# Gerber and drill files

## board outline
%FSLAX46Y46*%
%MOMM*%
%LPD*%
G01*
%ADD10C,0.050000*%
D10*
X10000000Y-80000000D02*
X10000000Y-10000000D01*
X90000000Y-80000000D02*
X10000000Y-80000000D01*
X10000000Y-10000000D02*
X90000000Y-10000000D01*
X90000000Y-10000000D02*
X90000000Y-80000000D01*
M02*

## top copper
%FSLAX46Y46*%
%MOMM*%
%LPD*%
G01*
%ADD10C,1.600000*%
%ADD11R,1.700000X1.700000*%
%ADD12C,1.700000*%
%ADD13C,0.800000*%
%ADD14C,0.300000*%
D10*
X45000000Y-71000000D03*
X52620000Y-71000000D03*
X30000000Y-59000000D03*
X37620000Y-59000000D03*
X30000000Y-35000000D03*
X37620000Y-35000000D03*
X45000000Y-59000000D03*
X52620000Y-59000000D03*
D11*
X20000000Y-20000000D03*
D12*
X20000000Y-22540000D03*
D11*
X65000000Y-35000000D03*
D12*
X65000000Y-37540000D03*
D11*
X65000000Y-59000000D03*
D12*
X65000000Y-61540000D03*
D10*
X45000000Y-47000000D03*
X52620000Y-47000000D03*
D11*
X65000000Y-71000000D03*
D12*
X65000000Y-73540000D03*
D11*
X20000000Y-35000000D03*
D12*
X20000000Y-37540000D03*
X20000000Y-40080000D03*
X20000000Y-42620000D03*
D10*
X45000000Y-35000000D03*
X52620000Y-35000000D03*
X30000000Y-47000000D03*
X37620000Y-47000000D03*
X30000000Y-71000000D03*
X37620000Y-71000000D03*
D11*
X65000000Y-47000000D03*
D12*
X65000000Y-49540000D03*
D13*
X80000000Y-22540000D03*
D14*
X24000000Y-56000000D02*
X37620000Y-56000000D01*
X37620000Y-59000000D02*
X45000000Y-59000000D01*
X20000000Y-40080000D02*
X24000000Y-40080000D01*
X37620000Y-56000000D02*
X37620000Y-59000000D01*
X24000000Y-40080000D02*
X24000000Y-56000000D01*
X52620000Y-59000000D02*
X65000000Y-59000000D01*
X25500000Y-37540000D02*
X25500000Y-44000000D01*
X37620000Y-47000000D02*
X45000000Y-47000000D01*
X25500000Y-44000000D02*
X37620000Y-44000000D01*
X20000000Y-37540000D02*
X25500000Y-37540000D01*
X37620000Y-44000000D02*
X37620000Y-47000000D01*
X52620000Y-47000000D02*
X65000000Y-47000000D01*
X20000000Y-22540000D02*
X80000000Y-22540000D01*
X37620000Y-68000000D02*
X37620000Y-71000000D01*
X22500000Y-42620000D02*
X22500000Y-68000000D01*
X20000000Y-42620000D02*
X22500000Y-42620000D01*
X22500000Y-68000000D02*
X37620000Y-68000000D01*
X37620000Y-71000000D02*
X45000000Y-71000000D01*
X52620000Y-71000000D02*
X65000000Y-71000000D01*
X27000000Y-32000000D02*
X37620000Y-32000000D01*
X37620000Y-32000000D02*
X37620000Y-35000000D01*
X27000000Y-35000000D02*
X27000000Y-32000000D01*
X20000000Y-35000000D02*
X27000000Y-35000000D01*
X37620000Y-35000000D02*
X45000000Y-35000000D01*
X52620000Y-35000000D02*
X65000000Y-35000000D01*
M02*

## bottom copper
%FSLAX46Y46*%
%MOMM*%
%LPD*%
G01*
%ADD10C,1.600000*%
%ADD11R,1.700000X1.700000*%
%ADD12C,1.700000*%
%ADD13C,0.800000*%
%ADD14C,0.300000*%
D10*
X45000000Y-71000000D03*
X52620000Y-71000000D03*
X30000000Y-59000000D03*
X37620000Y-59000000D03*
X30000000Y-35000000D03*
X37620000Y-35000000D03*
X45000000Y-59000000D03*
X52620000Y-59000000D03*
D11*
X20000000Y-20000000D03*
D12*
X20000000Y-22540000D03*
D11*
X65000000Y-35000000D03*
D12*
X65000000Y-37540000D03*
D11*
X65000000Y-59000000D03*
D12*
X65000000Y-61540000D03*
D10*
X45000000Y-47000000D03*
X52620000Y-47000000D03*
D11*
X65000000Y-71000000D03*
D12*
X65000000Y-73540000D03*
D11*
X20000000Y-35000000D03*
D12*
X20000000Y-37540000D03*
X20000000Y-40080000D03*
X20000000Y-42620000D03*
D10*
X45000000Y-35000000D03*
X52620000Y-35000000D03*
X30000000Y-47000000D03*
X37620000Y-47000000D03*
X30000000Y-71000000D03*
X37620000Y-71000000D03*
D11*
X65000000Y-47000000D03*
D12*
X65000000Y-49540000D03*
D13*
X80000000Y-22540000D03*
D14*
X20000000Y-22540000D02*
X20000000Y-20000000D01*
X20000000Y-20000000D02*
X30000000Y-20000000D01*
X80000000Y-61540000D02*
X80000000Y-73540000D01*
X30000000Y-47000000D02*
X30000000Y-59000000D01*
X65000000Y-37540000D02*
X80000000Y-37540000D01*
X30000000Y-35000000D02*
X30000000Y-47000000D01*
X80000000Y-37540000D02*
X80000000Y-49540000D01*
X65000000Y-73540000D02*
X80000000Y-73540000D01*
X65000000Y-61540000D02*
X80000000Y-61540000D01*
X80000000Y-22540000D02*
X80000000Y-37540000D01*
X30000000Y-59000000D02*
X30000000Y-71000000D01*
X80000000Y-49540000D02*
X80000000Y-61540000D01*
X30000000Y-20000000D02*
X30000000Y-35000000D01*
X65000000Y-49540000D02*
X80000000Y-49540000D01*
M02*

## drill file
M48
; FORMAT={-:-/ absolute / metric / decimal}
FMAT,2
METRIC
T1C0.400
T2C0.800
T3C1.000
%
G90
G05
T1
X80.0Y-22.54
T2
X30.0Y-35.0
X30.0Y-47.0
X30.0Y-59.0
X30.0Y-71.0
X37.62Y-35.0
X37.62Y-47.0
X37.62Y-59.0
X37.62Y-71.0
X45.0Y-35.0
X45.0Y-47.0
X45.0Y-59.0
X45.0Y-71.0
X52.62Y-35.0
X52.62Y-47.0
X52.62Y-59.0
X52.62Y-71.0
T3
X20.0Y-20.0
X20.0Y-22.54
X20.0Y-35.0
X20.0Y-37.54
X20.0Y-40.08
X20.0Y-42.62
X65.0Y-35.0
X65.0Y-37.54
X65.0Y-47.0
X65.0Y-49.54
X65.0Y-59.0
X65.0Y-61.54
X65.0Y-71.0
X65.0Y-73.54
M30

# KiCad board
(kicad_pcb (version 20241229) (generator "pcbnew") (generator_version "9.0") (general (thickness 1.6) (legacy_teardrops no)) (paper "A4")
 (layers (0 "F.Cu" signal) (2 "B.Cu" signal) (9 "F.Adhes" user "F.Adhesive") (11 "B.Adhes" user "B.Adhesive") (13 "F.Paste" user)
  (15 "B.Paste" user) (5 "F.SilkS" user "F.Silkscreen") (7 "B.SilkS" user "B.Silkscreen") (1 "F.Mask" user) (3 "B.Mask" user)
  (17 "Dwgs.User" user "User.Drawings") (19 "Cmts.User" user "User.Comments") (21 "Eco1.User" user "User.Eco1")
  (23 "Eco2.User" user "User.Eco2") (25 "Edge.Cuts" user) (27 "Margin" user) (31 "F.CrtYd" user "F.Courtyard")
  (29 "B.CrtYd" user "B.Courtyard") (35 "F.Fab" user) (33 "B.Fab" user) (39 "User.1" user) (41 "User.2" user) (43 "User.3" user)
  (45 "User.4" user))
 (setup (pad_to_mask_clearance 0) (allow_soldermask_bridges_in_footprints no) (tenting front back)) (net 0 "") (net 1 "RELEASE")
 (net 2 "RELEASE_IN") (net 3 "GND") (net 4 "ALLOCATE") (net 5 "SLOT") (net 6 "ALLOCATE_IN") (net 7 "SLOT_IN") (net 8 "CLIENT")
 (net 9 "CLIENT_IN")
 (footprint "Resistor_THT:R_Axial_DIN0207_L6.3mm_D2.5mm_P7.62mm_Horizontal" (layer "F.Cu") (at 45 71)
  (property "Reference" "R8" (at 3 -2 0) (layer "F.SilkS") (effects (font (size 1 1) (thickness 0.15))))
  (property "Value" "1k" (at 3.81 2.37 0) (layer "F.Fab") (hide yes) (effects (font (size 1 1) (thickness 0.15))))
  (pad "1" thru_hole circle (at 0 0) (size 1.6 1.6) (drill 0.8) (layers "*.Cu" "*.Mask") (remove_unused_layers no) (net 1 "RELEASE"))
  (pad "2" thru_hole circle (at 7.62 0) (size 1.6 1.6) (drill 0.8) (layers "*.Cu" "*.Mask") (remove_unused_layers no) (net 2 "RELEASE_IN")))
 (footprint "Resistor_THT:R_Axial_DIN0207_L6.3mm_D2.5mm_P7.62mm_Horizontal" (layer "F.Cu") (at 30 59)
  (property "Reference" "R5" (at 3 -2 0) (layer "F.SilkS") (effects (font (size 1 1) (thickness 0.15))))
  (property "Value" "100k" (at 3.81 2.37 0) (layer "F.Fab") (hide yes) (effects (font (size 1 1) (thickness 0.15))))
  (pad "1" thru_hole circle (at 0 0) (size 1.6 1.6) (drill 0.8) (layers "*.Cu" "*.Mask") (remove_unused_layers no) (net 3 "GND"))
  (pad "2" thru_hole circle (at 7.62 0) (size 1.6 1.6) (drill 0.8) (layers "*.Cu" "*.Mask") (remove_unused_layers no) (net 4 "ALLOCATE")))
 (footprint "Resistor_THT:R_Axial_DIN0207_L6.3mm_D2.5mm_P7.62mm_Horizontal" (layer "F.Cu") (at 30 35)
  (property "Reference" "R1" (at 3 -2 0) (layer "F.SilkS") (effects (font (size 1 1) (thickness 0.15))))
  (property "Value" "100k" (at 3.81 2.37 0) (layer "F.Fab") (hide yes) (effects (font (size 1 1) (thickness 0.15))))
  (pad "1" thru_hole circle (at 0 0) (size 1.6 1.6) (drill 0.8) (layers "*.Cu" "*.Mask") (remove_unused_layers no) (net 3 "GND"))
  (pad "2" thru_hole circle (at 7.62 0) (size 1.6 1.6) (drill 0.8) (layers "*.Cu" "*.Mask") (remove_unused_layers no) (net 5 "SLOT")))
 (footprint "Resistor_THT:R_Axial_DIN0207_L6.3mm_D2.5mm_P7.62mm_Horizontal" (layer "F.Cu") (at 45 59)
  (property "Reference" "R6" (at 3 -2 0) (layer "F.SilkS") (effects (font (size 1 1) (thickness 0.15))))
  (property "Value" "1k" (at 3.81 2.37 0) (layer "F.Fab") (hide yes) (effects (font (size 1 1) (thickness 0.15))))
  (pad "1" thru_hole circle (at 0 0) (size 1.6 1.6) (drill 0.8) (layers "*.Cu" "*.Mask") (remove_unused_layers no) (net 4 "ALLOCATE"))
  (pad "2" thru_hole circle (at 7.62 0) (size 1.6 1.6) (drill 0.8) (layers "*.Cu" "*.Mask") (remove_unused_layers no) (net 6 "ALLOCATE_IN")))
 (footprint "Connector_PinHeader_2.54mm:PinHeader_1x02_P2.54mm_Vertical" (layer "F.Cu") (at 20 20)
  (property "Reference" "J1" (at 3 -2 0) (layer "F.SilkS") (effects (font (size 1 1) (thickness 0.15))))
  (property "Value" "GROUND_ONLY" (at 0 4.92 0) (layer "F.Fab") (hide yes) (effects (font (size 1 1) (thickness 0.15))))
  (pad "1" thru_hole rect (at 0 0) (size 1.7 1.7) (drill 1) (layers "*.Cu" "*.Mask") (remove_unused_layers no) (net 3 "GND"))
  (pad "2" thru_hole circle (at 0 2.54) (size 1.7 1.7) (drill 1) (layers "*.Cu" "*.Mask") (remove_unused_layers no) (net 3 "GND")))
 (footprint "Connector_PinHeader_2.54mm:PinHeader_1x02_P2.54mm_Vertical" (layer "F.Cu") (at 65 35)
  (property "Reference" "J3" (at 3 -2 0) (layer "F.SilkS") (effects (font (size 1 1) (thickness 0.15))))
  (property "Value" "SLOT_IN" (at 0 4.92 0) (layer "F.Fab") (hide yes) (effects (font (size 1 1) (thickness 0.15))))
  (pad "1" thru_hole rect (at 0 0) (size 1.7 1.7) (drill 1) (layers "*.Cu" "*.Mask") (remove_unused_layers no) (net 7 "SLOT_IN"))
  (pad "2" thru_hole circle (at 0 2.54) (size 1.7 1.7) (drill 1) (layers "*.Cu" "*.Mask") (remove_unused_layers no) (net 3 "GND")))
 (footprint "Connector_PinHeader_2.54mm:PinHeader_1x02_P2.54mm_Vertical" (layer "F.Cu") (at 65 59)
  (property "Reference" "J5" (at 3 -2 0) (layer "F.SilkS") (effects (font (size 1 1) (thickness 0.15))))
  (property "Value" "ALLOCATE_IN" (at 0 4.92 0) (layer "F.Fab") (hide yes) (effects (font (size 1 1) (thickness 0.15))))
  (pad "1" thru_hole rect (at 0 0) (size 1.7 1.7) (drill 1) (layers "*.Cu" "*.Mask") (remove_unused_layers no) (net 6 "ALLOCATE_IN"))
  (pad "2" thru_hole circle (at 0 2.54) (size 1.7 1.7) (drill 1) (layers "*.Cu" "*.Mask") (remove_unused_layers no) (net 3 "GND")))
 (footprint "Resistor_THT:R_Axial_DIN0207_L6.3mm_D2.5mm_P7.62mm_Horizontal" (layer "F.Cu") (at 45 47)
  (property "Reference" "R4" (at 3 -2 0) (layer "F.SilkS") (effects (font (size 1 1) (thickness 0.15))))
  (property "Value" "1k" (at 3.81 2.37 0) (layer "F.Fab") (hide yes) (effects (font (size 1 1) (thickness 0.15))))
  (pad "1" thru_hole circle (at 0 0) (size 1.6 1.6) (drill 0.8) (layers "*.Cu" "*.Mask") (remove_unused_layers no) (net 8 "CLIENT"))
  (pad "2" thru_hole circle (at 7.62 0) (size 1.6 1.6) (drill 0.8) (layers "*.Cu" "*.Mask") (remove_unused_layers no) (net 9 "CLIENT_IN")))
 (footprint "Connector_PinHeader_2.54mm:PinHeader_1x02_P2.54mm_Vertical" (layer "F.Cu") (at 65 71)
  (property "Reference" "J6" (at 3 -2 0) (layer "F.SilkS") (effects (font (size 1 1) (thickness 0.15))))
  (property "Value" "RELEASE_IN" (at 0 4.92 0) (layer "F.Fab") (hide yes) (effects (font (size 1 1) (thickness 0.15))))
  (pad "1" thru_hole rect (at 0 0) (size 1.7 1.7) (drill 1) (layers "*.Cu" "*.Mask") (remove_unused_layers no) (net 2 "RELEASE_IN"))
  (pad "2" thru_hole circle (at 0 2.54) (size 1.7 1.7) (drill 1) (layers "*.Cu" "*.Mask") (remove_unused_layers no) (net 3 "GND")))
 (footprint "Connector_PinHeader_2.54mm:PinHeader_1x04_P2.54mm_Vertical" (layer "F.Cu") (at 20 35)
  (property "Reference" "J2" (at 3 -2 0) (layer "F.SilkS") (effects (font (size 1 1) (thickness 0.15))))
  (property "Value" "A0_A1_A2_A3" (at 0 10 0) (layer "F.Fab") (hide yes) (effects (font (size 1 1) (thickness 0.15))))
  (pad "1" thru_hole rect (at 0 0) (size 1.7 1.7) (drill 1) (layers "*.Cu" "*.Mask") (remove_unused_layers no) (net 5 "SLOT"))
  (pad "2" thru_hole circle (at 0 2.54) (size 1.7 1.7) (drill 1) (layers "*.Cu" "*.Mask") (remove_unused_layers no) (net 8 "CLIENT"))
  (pad "3" thru_hole circle (at 0 5.08) (size 1.7 1.7) (drill 1) (layers "*.Cu" "*.Mask") (remove_unused_layers no) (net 4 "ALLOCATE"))
  (pad "4" thru_hole circle (at 0 7.62) (size 1.7 1.7) (drill 1) (layers "*.Cu" "*.Mask") (remove_unused_layers no) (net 1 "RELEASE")))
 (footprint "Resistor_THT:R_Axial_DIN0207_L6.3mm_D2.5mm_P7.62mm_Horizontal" (layer "F.Cu") (at 45 35)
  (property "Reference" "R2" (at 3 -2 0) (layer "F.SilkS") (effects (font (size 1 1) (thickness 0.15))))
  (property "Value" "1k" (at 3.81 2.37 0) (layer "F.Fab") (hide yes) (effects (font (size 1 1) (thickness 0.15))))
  (pad "1" thru_hole circle (at 0 0) (size 1.6 1.6) (drill 0.8) (layers "*.Cu" "*.Mask") (remove_unused_layers no) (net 5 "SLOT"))
  (pad "2" thru_hole circle (at 7.62 0) (size 1.6 1.6) (drill 0.8) (layers "*.Cu" "*.Mask") (remove_unused_layers no) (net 7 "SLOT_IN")))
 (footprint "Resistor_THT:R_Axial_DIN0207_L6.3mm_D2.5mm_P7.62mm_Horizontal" (layer "F.Cu") (at 30 47)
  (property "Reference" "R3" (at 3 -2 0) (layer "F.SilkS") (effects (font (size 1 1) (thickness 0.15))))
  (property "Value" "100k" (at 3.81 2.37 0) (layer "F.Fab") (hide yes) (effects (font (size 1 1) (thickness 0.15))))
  (pad "1" thru_hole circle (at 0 0) (size 1.6 1.6) (drill 0.8) (layers "*.Cu" "*.Mask") (remove_unused_layers no) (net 3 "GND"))
  (pad "2" thru_hole circle (at 7.62 0) (size 1.6 1.6) (drill 0.8) (layers "*.Cu" "*.Mask") (remove_unused_layers no) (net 8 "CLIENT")))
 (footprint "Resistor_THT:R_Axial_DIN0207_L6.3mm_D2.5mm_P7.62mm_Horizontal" (layer "F.Cu") (at 30 71)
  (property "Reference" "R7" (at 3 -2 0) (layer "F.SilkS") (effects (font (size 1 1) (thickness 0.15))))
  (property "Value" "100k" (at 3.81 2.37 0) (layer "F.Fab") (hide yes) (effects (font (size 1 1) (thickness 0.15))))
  (pad "1" thru_hole circle (at 0 0) (size 1.6 1.6) (drill 0.8) (layers "*.Cu" "*.Mask") (remove_unused_layers no) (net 3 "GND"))
  (pad "2" thru_hole circle (at 7.62 0) (size 1.6 1.6) (drill 0.8) (layers "*.Cu" "*.Mask") (remove_unused_layers no) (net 1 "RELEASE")))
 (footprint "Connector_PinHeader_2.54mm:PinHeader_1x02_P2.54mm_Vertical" (layer "F.Cu") (at 65 47)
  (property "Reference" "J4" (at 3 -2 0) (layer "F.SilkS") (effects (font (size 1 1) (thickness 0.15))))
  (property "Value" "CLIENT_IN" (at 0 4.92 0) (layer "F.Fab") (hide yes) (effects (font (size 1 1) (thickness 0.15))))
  (pad "1" thru_hole rect (at 0 0) (size 1.7 1.7) (drill 1) (layers "*.Cu" "*.Mask") (remove_unused_layers no) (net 9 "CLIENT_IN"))
  (pad "2" thru_hole circle (at 0 2.54) (size 1.7 1.7) (drill 1) (layers "*.Cu" "*.Mask") (remove_unused_layers no) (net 3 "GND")))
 (gr_line (start 10 80) (end 10 10) (stroke (width 0.05) (type default)) (layer "Edge.Cuts"))
 (gr_line (start 90 80) (end 10 80) (stroke (width 0.05) (type default)) (layer "Edge.Cuts"))
 (gr_line (start 10 10) (end 90 10) (stroke (width 0.05) (type default)) (layer "Edge.Cuts"))
 (gr_line (start 90 10) (end 90 80) (stroke (width 0.05) (type default)) (layer "Edge.Cuts"))
 (segment (start 24 56) (end 37.62 56) (width 0.3) (layer "F.Cu") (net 4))
 (segment (start 37.62 59) (end 45 59) (width 0.3) (layer "F.Cu") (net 4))
 (segment (start 20 40.08) (end 24 40.08) (width 0.3) (layer "F.Cu") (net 4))
 (segment (start 37.62 56) (end 37.62 59) (width 0.3) (layer "F.Cu") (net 4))
 (segment (start 24 40.08) (end 24 56) (width 0.3) (layer "F.Cu") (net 4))
 (segment (start 52.62 59) (end 65 59) (width 0.3) (layer "F.Cu") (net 6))
 (segment (start 25.5 37.54) (end 25.5 44) (width 0.3) (layer "F.Cu") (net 8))
 (segment (start 37.62 47) (end 45 47) (width 0.3) (layer "F.Cu") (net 8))
 (segment (start 25.5 44) (end 37.62 44) (width 0.3) (layer "F.Cu") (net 8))
 (segment (start 20 37.54) (end 25.5 37.54) (width 0.3) (layer "F.Cu") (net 8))
 (segment (start 37.62 44) (end 37.62 47) (width 0.3) (layer "F.Cu") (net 8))
 (segment (start 52.62 47) (end 65 47) (width 0.3) (layer "F.Cu") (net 9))
 (segment (start 20 22.54) (end 80 22.54) (width 0.3) (layer "F.Cu") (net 3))
 (via (at 80 22.54) (size 0.8) (drill 0.4) (layers "F.Cu" "B.Cu") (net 3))
 (segment (start 20 22.54) (end 20 20) (width 0.3) (layer "B.Cu") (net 3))
 (segment (start 20 20) (end 30 20) (width 0.3) (layer "B.Cu") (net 3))
 (segment (start 80 61.54) (end 80 73.54) (width 0.3) (layer "B.Cu") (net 3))
 (segment (start 30 47) (end 30 59) (width 0.3) (layer "B.Cu") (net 3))
 (segment (start 65 37.54) (end 80 37.54) (width 0.3) (layer "B.Cu") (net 3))
 (segment (start 30 35) (end 30 47) (width 0.3) (layer "B.Cu") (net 3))
 (segment (start 80 37.54) (end 80 49.54) (width 0.3) (layer "B.Cu") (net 3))
 (segment (start 65 73.54) (end 80 73.54) (width 0.3) (layer "B.Cu") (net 3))
 (segment (start 65 61.54) (end 80 61.54) (width 0.3) (layer "B.Cu") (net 3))
 (segment (start 80 22.54) (end 80 37.54) (width 0.3) (layer "B.Cu") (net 3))
 (segment (start 30 59) (end 30 71) (width 0.3) (layer "B.Cu") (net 3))
 (segment (start 80 49.54) (end 80 61.54) (width 0.3) (layer "B.Cu") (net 3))
 (segment (start 30 20) (end 30 35) (width 0.3) (layer "B.Cu") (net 3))
 (segment (start 65 49.54) (end 80 49.54) (width 0.3) (layer "B.Cu") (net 3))
 (segment (start 37.62 68) (end 37.62 71) (width 0.3) (layer "F.Cu") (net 1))
 (segment (start 22.5 42.62) (end 22.5 68) (width 0.3) (layer "F.Cu") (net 1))
 (segment (start 20 42.62) (end 22.5 42.62) (width 0.3) (layer "F.Cu") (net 1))
 (segment (start 22.5 68) (end 37.62 68) (width 0.3) (layer "F.Cu") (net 1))
 (segment (start 37.62 71) (end 45 71) (width 0.3) (layer "F.Cu") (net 1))
 (segment (start 52.62 71) (end 65 71) (width 0.3) (layer "F.Cu") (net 2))
 (segment (start 27 32) (end 37.62 32) (width 0.3) (layer "F.Cu") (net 5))
 (segment (start 37.62 32) (end 37.62 35) (width 0.3) (layer "F.Cu") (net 5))
 (segment (start 27 35) (end 27 32) (width 0.3) (layer "F.Cu") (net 5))
 (segment (start 20 35) (end 27 35) (width 0.3) (layer "F.Cu") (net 5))
 (segment (start 37.62 35) (end 45 35) (width 0.3) (layer "F.Cu") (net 5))
 (segment (start 52.62 35) (end 65 35) (width 0.3) (layer "F.Cu") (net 7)))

